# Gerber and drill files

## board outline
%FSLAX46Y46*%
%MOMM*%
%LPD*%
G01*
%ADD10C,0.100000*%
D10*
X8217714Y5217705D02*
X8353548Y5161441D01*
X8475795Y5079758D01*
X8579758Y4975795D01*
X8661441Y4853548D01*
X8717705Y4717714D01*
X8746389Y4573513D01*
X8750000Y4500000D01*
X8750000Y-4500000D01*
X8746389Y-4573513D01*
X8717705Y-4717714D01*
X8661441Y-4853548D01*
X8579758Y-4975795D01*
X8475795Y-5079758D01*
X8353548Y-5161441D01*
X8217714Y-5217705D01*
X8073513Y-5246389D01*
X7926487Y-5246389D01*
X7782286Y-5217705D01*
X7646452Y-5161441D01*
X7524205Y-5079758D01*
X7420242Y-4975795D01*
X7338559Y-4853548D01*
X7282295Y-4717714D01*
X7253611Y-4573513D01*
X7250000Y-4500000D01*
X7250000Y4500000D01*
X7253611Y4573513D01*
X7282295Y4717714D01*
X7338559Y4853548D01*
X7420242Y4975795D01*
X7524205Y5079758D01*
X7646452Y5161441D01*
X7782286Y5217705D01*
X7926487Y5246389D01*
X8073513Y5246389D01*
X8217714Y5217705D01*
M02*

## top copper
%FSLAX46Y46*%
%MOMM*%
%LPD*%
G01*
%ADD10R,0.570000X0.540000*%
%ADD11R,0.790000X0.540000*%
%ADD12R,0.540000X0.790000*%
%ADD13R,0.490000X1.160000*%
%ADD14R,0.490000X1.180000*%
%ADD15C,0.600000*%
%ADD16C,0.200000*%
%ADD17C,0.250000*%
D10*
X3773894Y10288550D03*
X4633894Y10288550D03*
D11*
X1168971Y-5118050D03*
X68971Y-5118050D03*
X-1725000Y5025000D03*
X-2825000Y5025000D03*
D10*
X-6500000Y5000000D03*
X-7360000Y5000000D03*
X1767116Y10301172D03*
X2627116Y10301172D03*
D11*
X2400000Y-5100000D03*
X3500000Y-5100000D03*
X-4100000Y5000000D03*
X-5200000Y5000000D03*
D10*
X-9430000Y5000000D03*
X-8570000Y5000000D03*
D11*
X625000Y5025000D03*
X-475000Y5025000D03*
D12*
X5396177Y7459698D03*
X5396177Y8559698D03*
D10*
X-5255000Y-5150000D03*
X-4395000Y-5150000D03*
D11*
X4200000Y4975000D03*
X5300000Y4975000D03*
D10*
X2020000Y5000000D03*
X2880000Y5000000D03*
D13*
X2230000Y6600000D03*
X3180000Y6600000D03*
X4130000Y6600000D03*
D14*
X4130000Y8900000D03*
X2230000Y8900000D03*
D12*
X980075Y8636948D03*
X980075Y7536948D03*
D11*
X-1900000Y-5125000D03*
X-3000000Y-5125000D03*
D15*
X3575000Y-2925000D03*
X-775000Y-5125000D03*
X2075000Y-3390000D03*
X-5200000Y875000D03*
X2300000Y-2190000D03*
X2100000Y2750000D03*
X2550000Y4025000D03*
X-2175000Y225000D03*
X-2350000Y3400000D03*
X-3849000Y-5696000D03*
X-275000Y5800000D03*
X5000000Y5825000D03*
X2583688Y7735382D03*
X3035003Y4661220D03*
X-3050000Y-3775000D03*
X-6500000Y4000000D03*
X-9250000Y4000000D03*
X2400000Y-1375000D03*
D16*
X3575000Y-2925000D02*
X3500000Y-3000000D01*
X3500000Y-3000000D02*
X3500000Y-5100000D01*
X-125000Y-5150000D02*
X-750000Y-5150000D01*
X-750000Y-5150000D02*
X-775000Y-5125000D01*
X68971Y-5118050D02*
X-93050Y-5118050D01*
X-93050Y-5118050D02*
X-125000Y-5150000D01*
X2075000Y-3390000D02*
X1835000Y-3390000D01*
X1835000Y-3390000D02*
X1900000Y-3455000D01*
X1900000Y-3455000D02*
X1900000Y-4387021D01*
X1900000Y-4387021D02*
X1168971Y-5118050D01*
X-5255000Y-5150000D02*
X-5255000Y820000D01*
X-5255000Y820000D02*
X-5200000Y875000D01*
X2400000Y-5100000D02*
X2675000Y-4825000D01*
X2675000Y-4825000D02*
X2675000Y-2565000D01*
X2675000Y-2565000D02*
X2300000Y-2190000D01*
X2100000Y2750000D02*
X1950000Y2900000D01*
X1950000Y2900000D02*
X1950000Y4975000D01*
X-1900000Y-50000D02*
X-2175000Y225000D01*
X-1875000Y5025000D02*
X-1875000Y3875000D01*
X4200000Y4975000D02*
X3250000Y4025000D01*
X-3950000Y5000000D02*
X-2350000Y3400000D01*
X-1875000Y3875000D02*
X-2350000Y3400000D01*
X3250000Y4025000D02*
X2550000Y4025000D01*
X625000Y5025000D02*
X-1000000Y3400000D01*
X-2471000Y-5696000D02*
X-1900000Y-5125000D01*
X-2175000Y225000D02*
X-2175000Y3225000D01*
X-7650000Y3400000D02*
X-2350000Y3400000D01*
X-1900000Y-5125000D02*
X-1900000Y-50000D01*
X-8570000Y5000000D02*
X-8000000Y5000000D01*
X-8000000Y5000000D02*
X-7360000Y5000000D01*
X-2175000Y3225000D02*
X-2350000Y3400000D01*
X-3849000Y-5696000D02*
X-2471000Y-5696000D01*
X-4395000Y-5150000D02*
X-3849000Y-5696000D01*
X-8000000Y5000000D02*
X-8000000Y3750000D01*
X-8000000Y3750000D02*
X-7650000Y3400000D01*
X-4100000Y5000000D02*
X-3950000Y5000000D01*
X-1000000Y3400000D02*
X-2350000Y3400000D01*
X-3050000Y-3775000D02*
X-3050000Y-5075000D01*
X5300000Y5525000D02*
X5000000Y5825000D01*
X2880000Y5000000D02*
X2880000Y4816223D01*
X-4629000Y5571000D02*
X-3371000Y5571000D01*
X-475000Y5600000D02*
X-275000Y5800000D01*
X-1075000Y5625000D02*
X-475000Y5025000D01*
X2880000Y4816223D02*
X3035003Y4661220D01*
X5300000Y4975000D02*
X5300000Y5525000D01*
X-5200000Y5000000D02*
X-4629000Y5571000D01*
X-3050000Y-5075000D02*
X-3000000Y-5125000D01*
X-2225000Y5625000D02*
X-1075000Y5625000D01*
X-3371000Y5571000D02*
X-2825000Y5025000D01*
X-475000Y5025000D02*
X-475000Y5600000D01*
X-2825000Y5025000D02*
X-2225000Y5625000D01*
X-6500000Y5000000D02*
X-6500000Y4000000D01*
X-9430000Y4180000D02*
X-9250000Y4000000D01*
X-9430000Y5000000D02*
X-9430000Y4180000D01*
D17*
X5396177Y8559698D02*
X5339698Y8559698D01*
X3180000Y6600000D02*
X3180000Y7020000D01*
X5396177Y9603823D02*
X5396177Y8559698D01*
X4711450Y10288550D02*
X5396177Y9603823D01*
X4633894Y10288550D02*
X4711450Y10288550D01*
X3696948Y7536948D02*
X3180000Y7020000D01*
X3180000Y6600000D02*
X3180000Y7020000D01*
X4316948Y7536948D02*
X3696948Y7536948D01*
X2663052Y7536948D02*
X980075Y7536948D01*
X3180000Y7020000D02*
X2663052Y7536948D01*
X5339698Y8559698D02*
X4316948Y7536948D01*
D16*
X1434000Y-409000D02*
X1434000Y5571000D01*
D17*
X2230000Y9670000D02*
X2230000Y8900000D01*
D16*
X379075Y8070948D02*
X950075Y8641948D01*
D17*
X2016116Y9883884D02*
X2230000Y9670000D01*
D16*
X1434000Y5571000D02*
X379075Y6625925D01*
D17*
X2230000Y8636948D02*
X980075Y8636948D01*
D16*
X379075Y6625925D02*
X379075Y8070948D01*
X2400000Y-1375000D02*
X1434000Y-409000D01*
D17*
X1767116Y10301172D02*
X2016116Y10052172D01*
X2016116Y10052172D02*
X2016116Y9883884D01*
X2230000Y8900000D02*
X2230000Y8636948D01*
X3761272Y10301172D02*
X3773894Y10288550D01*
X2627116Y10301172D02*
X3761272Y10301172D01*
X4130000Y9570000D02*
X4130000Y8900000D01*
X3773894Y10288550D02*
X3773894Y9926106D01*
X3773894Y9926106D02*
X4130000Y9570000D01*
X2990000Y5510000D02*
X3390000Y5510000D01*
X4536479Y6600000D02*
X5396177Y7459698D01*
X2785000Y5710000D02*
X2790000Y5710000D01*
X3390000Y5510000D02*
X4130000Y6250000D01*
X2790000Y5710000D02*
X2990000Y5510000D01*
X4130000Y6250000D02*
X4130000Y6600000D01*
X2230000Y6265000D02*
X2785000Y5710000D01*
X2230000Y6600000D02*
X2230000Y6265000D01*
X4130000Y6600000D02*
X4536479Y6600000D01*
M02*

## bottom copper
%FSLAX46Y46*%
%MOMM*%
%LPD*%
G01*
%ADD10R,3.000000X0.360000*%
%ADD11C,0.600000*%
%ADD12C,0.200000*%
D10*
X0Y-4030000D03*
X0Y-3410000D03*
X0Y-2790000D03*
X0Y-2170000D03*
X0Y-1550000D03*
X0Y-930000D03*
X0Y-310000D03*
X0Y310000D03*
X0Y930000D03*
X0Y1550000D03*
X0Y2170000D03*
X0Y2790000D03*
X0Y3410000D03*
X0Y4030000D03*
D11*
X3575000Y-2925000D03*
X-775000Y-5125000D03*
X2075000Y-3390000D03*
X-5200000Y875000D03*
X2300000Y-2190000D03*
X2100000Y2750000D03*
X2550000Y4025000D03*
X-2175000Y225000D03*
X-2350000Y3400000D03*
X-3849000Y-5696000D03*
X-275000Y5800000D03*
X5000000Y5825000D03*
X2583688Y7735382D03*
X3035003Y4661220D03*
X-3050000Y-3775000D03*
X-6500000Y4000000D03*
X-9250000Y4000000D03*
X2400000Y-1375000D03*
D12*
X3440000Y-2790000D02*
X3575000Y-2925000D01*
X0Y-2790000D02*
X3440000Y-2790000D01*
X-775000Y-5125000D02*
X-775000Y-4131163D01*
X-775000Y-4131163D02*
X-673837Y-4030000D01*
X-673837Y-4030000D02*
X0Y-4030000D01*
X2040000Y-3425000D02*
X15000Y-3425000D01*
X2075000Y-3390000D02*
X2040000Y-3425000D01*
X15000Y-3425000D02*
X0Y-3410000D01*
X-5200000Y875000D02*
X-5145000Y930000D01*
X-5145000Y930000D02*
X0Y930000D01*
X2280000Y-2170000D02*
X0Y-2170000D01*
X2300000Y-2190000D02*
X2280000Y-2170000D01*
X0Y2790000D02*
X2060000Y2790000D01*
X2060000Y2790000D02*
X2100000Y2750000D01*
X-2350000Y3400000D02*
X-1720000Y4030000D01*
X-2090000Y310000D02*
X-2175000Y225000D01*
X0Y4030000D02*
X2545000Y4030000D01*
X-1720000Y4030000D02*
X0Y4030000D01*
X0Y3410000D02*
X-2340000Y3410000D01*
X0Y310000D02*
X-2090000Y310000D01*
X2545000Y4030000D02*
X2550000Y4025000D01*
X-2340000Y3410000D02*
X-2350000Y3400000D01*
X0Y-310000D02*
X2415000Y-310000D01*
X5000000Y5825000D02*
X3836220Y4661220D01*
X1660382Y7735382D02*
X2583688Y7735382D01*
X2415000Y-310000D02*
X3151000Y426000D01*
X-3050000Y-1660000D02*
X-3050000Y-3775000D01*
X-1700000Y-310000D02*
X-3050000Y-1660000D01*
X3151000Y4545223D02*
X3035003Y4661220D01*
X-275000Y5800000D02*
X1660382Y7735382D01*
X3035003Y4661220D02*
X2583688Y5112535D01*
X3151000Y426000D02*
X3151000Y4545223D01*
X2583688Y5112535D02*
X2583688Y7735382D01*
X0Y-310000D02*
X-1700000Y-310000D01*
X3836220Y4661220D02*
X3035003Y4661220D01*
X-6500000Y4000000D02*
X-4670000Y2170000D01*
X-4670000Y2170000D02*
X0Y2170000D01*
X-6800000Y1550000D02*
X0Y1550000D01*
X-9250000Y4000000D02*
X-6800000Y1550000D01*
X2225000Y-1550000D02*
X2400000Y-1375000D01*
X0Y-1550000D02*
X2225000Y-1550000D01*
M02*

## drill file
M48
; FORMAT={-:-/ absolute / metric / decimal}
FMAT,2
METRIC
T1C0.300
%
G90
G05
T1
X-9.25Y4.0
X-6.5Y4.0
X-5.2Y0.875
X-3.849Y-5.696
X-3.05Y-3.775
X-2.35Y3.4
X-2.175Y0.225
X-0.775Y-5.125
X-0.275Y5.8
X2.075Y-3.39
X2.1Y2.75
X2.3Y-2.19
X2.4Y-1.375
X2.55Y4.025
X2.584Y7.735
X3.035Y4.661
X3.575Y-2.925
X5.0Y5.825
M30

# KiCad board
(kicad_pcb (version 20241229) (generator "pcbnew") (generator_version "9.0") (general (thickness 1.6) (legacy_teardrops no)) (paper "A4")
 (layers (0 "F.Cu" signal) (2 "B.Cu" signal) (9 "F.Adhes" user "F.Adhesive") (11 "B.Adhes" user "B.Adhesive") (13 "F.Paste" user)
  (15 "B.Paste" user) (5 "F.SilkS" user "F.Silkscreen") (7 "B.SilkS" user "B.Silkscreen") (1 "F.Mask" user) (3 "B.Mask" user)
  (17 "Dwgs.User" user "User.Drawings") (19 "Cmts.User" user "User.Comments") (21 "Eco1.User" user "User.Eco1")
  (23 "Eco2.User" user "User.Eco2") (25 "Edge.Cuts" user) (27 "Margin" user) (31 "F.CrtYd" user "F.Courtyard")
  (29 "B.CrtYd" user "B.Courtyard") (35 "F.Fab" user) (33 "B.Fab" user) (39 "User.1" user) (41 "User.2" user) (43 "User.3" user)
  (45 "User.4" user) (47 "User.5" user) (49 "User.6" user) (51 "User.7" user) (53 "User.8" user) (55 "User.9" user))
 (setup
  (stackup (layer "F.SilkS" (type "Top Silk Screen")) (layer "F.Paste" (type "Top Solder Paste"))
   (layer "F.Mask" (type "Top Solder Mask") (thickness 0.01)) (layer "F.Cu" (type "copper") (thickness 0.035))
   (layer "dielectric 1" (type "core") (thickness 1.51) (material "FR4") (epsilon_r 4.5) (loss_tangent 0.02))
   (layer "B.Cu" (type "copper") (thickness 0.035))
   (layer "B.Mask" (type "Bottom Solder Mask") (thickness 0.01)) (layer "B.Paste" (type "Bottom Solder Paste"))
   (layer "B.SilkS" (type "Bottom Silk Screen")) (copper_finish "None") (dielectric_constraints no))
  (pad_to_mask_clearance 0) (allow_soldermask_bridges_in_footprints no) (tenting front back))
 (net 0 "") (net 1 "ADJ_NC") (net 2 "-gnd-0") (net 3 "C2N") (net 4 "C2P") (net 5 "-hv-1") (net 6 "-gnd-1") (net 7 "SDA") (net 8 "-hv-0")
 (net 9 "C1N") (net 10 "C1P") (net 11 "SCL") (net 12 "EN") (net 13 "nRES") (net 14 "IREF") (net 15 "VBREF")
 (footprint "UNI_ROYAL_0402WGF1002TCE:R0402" (layer "F.Cu") (at 4.203894 -10.28855)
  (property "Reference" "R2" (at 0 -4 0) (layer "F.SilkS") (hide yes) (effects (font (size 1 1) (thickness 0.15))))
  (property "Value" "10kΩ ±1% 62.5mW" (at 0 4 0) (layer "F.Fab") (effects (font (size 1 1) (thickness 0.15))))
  (pad "1" smd rect (at -0.43 0) (size 0.57 0.54) (layers "F.Cu" "F.Mask" "F.Paste") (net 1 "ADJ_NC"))
  (pad "2" smd rect (at 0.43 0) (size 0.57 0.54) (layers "F.Cu" "F.Mask" "F.Paste") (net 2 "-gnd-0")))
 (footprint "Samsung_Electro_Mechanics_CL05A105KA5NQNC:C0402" (layer "F.Cu") (at 0.618971 5.11805 180)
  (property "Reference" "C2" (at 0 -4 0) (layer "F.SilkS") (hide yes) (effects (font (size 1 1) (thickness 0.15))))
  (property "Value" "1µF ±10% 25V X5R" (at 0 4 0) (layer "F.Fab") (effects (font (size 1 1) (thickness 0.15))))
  (pad "1" smd rect (at -0.55 0 180) (size 0.79 0.54) (layers "F.Cu" "F.Mask" "F.Paste") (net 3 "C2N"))
  (pad "2" smd rect (at 0.55 0 180) (size 0.79 0.54) (layers "F.Cu" "F.Mask" "F.Paste") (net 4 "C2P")))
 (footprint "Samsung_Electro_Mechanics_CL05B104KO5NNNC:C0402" (layer "F.Cu") (at -2.275 -5.025 180)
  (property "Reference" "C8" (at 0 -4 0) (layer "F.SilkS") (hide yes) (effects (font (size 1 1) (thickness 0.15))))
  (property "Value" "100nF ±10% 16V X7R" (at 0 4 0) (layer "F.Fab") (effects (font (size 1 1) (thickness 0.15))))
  (pad "1" smd rect (at -0.55 0 180) (size 0.79 0.54) (layers "F.Cu" "F.Mask" "F.Paste") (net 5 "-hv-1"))
  (pad "2" smd rect (at 0.55 0 180) (size 0.79 0.54) (layers "F.Cu" "F.Mask" "F.Paste") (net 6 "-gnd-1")))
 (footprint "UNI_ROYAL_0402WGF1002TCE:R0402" (layer "F.Cu") (at -6.93 -5 180)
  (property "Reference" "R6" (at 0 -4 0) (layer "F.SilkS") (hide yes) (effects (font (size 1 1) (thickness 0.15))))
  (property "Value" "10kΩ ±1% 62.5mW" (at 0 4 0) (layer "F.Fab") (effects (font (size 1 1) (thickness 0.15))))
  (pad "1" smd rect (at -0.43 0 180) (size 0.57 0.54) (layers "F.Cu" "F.Mask" "F.Paste") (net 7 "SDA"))
  (pad "2" smd rect (at 0.43 0 180) (size 0.57 0.54) (layers "F.Cu" "F.Mask" "F.Paste") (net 5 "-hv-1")))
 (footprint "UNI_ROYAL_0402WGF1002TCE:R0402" (layer "F.Cu") (at 2.197116 -10.301172)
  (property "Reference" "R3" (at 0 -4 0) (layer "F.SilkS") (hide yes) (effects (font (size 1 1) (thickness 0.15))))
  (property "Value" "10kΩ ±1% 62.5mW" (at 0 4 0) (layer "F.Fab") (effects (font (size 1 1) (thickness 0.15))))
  (pad "1" smd rect (at -0.43 0) (size 0.57 0.54) (layers "F.Cu" "F.Mask" "F.Paste") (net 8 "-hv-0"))
  (pad "2" smd rect (at 0.43 0) (size 0.57 0.54) (layers "F.Cu" "F.Mask" "F.Paste") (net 1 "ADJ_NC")))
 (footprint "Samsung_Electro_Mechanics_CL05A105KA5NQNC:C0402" (layer "F.Cu") (at 2.95 5.1)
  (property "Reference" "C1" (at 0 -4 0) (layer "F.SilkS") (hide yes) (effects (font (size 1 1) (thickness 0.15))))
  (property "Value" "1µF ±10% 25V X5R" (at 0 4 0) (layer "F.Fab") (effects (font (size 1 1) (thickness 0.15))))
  (pad "1" smd rect (at -0.55 0) (size 0.79 0.54) (layers "F.Cu" "F.Mask" "F.Paste") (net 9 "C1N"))
  (pad "2" smd rect (at 0.55 0) (size 0.79 0.54) (layers "F.Cu" "F.Mask" "F.Paste") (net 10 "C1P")))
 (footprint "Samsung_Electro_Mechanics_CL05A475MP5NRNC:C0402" (layer "F.Cu") (at -4.65 -5 180)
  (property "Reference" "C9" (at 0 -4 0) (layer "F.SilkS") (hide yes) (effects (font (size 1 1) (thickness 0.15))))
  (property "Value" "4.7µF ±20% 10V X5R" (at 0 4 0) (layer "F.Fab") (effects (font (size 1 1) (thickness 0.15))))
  (pad "1" smd rect (at -0.55 0 180) (size 0.79 0.54) (layers "F.Cu" "F.Mask" "F.Paste") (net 5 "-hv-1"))
  (pad "2" smd rect (at 0.55 0 180) (size 0.79 0.54) (layers "F.Cu" "F.Mask" "F.Paste") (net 6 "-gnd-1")))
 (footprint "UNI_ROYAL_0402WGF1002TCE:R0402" (layer "F.Cu") (at -9 -5)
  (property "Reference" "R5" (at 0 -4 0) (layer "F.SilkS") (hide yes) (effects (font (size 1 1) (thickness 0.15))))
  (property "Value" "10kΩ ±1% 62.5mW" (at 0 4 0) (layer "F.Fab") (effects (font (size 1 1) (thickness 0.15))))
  (pad "1" smd rect (at -0.43 0) (size 0.57 0.54) (layers "F.Cu" "F.Mask" "F.Paste") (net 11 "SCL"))
  (pad "2" smd rect (at 0.43 0) (size 0.57 0.54) (layers "F.Cu" "F.Mask" "F.Paste") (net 5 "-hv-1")))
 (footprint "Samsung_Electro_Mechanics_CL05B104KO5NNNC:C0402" (layer "F.Cu") (at 0.075 -5.025 180)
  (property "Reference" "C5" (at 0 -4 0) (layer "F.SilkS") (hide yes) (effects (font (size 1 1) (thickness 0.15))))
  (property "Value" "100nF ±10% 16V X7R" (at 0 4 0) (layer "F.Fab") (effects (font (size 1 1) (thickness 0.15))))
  (pad "1" smd rect (at -0.55 0 180) (size 0.79 0.54) (layers "F.Cu" "F.Mask" "F.Paste") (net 5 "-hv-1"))
  (pad "2" smd rect (at 0.55 0 180) (size 0.79 0.54) (layers "F.Cu" "F.Mask" "F.Paste") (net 6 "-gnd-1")))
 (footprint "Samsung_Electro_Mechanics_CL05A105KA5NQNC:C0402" (layer "F.Cu") (at 5.396177 -8.009698 90)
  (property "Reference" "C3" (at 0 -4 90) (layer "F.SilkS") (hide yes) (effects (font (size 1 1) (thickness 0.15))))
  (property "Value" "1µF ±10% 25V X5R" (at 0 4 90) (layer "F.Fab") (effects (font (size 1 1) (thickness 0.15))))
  (pad "1" smd rect (at -0.55 0 90) (size 0.79 0.54) (layers "F.Cu" "F.Mask" "F.Paste") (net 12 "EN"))
  (pad "2" smd rect (at 0.55 0 90) (size 0.79 0.54) (layers "F.Cu" "F.Mask" "F.Paste") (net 2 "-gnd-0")))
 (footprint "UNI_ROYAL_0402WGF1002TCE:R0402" (layer "F.Cu") (at -4.825 5.15)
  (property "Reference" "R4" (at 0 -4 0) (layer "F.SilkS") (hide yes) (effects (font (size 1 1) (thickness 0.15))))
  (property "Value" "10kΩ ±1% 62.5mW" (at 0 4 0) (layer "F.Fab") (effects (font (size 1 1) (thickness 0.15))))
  (pad "1" smd rect (at -0.43 0) (size 0.57 0.54) (layers "F.Cu" "F.Mask" "F.Paste") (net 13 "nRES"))
  (pad "2" smd rect (at 0.43 0) (size 0.57 0.54) (layers "F.Cu" "F.Mask" "F.Paste") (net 5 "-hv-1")))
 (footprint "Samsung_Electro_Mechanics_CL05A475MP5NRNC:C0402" (layer "F.Cu") (at 4.75 -4.975)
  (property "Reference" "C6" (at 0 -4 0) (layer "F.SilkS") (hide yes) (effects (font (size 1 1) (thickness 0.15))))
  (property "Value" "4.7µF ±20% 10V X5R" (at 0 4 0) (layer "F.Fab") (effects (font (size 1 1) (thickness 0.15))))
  (pad "1" smd rect (at -0.55 0) (size 0.79 0.54) (layers "F.Cu" "F.Mask" "F.Paste") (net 5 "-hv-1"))
  (pad "2" smd rect (at 0.55 0) (size 0.79 0.54) (layers "F.Cu" "F.Mask" "F.Paste") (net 6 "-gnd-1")))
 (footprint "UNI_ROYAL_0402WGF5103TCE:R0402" (layer "F.Cu") (at 2.45 -5)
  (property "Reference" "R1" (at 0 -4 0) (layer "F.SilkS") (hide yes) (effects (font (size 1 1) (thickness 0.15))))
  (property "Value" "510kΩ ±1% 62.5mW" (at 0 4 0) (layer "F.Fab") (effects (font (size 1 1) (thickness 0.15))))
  (pad "1" smd rect (at -0.43 0) (size 0.57 0.54) (layers "F.Cu" "F.Mask" "F.Paste") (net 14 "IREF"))
  (pad "2" smd rect (at 0.43 0) (size 0.57 0.54) (layers "F.Cu" "F.Mask" "F.Paste") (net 6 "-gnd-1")))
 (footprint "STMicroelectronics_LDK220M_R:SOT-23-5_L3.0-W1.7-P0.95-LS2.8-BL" (layer "F.Cu") (at 3.18 -7.75)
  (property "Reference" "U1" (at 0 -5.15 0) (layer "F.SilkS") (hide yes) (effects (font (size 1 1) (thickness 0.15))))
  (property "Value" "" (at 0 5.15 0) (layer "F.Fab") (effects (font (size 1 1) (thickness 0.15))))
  (pad "1" smd rect (at -0.95 1.15) (size 0.49 1.16) (layers "F.Cu" "F.Mask" "F.Paste") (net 12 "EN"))
  (pad "2" smd rect (at 0 1.15) (size 0.49 1.16) (layers "F.Cu" "F.Mask" "F.Paste") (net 2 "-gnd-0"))
  (pad "3" smd rect (at 0.95 1.15) (size 0.49 1.16) (layers "F.Cu" "F.Mask" "F.Paste") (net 12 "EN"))
  (pad "4" smd rect (at 0.95 -1.15) (size 0.49 1.18) (layers "F.Cu" "F.Mask" "F.Paste") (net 1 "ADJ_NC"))
  (pad "5" smd rect (at -0.95 -1.15) (size 0.49 1.18) (layers "F.Cu" "F.Mask" "F.Paste") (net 8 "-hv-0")))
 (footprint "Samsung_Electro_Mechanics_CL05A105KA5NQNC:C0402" (layer "F.Cu") (at 0.980075 -8.086948 -90)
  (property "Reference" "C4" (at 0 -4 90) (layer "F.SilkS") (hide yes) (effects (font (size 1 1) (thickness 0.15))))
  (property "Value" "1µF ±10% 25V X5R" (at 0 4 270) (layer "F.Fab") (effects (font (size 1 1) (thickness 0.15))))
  (pad "1" smd rect (at -0.55 0 270) (size 0.79 0.54) (layers "F.Cu" "F.Mask" "F.Paste") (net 8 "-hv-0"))
  (pad "2" smd rect (at 0.55 0 270) (size 0.79 0.54) (layers "F.Cu" "F.Mask" "F.Paste") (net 2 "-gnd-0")))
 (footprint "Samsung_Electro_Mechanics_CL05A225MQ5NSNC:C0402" (layer "F.Cu") (at -2.45 5.125 180)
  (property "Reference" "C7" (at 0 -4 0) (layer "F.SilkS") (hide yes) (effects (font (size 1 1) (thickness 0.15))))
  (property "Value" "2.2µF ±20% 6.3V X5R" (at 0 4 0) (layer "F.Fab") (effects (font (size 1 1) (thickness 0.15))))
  (pad "1" smd rect (at -0.55 0 180) (size 0.79 0.54) (layers "F.Cu" "F.Mask" "F.Paste") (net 5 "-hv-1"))
  (pad "2" smd rect (at 0.55 0 180) (size 0.79 0.54) (layers "F.Cu" "F.Mask" "F.Paste") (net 6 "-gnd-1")))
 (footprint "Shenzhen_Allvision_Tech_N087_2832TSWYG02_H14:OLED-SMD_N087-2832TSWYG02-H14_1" (layer "F.Cu") (at 0 0)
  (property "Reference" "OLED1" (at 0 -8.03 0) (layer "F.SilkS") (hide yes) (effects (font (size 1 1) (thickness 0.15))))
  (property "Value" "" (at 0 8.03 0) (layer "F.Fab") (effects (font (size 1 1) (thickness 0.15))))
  (fp_poly
   (pts (xy 8.217714 -5.217705) (xy 8.353548 -5.161441) (xy 8.475795 -5.079758) (xy 8.579758 -4.975795) (xy 8.661441 -4.853548)
    (xy 8.717705 -4.717714) (xy 8.746389 -4.573513) (xy 8.75 -4.5) (xy 8.75 4.5) (xy 8.746389 4.573513) (xy 8.717705 4.717714)
    (xy 8.661441 4.853548) (xy 8.579758 4.975795) (xy 8.475795 5.079758) (xy 8.353548 5.161441) (xy 8.217714 5.217705)
    (xy 8.073513 5.246389) (xy 7.926487 5.246389) (xy 7.782286 5.217705) (xy 7.646452 5.161441) (xy 7.524205 5.079758)
    (xy 7.420242 4.975795) (xy 7.338559 4.853548) (xy 7.282295 4.717714) (xy 7.253611 4.573513) (xy 7.25 4.5) (xy 7.25 -4.5)
    (xy 7.253611 -4.573513) (xy 7.282295 -4.717714) (xy 7.338559 -4.853548) (xy 7.420242 -4.975795) (xy 7.524205 -5.079758)
    (xy 7.646452 -5.161441) (xy 7.782286 -5.217705) (xy 7.926487 -5.246389) (xy 8.073513 -5.246389))
   (stroke (width 0.1) (type solid)) (fill no) (layer "Edge.Cuts"))
  (pad "1" smd rect (at 0 4.03) (size 3 0.36) (layers "B.Cu" "B.Mask" "B.Paste") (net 4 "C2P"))
  (pad "2" smd rect (at 0 3.41) (size 3 0.36) (layers "B.Cu" "B.Mask" "B.Paste") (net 3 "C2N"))
  (pad "3" smd rect (at 0 2.79) (size 3 0.36) (layers "B.Cu" "B.Mask" "B.Paste") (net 10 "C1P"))
  (pad "4" smd rect (at 0 2.17) (size 3 0.36) (layers "B.Cu" "B.Mask" "B.Paste") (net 9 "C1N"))
  (pad "5" smd rect (at 0 1.55) (size 3 0.36) (layers "B.Cu" "B.Mask" "B.Paste") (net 8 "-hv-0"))
  (pad "6" smd rect (at 0 0.93) (size 3 0.36) (layers "B.Cu" "B.Mask" "B.Paste") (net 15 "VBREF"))
  (pad "7" smd rect (at 0 0.31) (size 3 0.36) (layers "B.Cu" "B.Mask" "B.Paste") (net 6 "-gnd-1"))
  (pad "8" smd rect (at 0 -0.31) (size 3 0.36) (layers "B.Cu" "B.Mask" "B.Paste") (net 5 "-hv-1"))
  (pad "9" smd rect (at 0 -0.93) (size 3 0.36) (layers "B.Cu" "B.Mask" "B.Paste") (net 13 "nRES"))
  (pad "10" smd rect (at 0 -1.55) (size 3 0.36) (layers "B.Cu" "B.Mask" "B.Paste") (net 11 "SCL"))
  (pad "11" smd rect (at 0 -2.17) (size 3 0.36) (layers "B.Cu" "B.Mask" "B.Paste") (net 7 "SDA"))
  (pad "12" smd rect (at 0 -2.79) (size 3 0.36) (layers "B.Cu" "B.Mask" "B.Paste") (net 14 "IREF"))
  (pad "13" smd rect (at 0 -3.41) (size 3 0.36) (layers "B.Cu" "B.Mask" "B.Paste") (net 5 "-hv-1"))
  (pad "14" smd rect (at 0 -4.03) (size 3 0.36) (layers "B.Cu" "B.Mask" "B.Paste") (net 5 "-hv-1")))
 (segment (start 3.575 2.925) (end 3.5 3) (width 0.2) (layer "F.Cu") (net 10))
 (segment (start 3.5 3) (end 3.5 5.1) (width 0.2) (layer "F.Cu") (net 10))
 (via (at 3.575 2.925) (size 0.6) (drill 0.3) (layers "F.Cu" "B.Cu") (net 10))
 (segment (start 3.44 2.79) (end 3.575 2.925) (width 0.2) (layer "B.Cu") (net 10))
 (segment (start 0 2.79) (end 3.44 2.79) (width 0.2) (layer "B.Cu") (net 10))
 (segment (start -0.125 5.15) (end -0.75 5.15) (width 0.2) (layer "F.Cu") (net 4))
 (segment (start -0.75 5.15) (end -0.775 5.125) (width 0.2) (layer "F.Cu") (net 4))
 (segment (start 0.068971 5.11805) (end -0.09305 5.11805) (width 0.2) (layer "F.Cu") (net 4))
 (segment (start -0.09305 5.11805) (end -0.125 5.15) (width 0.2) (layer "F.Cu") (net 4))
 (via (at -0.775 5.125) (size 0.6) (drill 0.3) (layers "F.Cu" "B.Cu") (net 4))
 (segment (start -0.775 5.125) (end -0.775 4.131163) (width 0.2) (layer "B.Cu") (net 4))
 (segment (start -0.775 4.131163) (end -0.673837 4.03) (width 0.2) (layer "B.Cu") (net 4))
 (segment (start -0.673837 4.03) (end 0 4.03) (width 0.2) (layer "B.Cu") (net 4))
 (segment (start 2.075 3.39) (end 1.835 3.39) (width 0.2) (layer "F.Cu") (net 3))
 (segment (start 1.835 3.39) (end 1.9 3.455) (width 0.2) (layer "F.Cu") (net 3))
 (segment (start 1.9 3.455) (end 1.9 4.387021) (width 0.2) (layer "F.Cu") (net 3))
 (segment (start 1.9 4.387021) (end 1.168971 5.11805) (width 0.2) (layer "F.Cu") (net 3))
 (via (at 2.075 3.39) (size 0.6) (drill 0.3) (layers "F.Cu" "B.Cu") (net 3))
 (segment (start 2.04 3.425) (end 0.015 3.425) (width 0.2) (layer "B.Cu") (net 3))
 (segment (start 2.075 3.39) (end 2.04 3.425) (width 0.2) (layer "B.Cu") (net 3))
 (segment (start 0.015 3.425) (end 0 3.41) (width 0.2) (layer "B.Cu") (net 3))
 (segment (start -5.255 5.15) (end -5.255 -0.82) (width 0.2) (layer "F.Cu") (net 13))
 (segment (start -5.255 -0.82) (end -5.2 -0.875) (width 0.2) (layer "F.Cu") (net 13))
 (via (at -5.2 -0.875) (size 0.6) (drill 0.3) (layers "F.Cu" "B.Cu") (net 13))
 (segment (start -5.2 -0.875) (end -5.145 -0.93) (width 0.2) (layer "B.Cu") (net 13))
 (segment (start -5.145 -0.93) (end 0 -0.93) (width 0.2) (layer "B.Cu") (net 13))
 (segment (start 2.4 5.1) (end 2.675 4.825) (width 0.2) (layer "F.Cu") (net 9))
 (segment (start 2.675 4.825) (end 2.675 2.565) (width 0.2) (layer "F.Cu") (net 9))
 (segment (start 2.675 2.565) (end 2.3 2.19) (width 0.2) (layer "F.Cu") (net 9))
 (via (at 2.3 2.19) (size 0.6) (drill 0.3) (layers "F.Cu" "B.Cu") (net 9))
 (segment (start 2.28 2.17) (end 0 2.17) (width 0.2) (layer "B.Cu") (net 9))
 (segment (start 2.3 2.19) (end 2.28 2.17) (width 0.2) (layer "B.Cu") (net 9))
 (segment (start 2.1 -2.75) (end 1.95 -2.9) (width 0.2) (layer "F.Cu") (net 14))
 (segment (start 1.95 -2.9) (end 1.95 -4.975) (width 0.2) (layer "F.Cu") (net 14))
 (via (at 2.1 -2.75) (size 0.6) (drill 0.3) (layers "F.Cu" "B.Cu") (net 14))
 (segment (start 0 -2.79) (end 2.06 -2.79) (width 0.2) (layer "B.Cu") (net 14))
 (segment (start 2.06 -2.79) (end 2.1 -2.75) (width 0.2) (layer "B.Cu") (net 14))
 (segment (start -1.9 0.05) (end -2.175 -0.225) (width 0.2) (layer "F.Cu") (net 5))
 (segment (start -1.875 -5.025) (end -1.875 -3.875) (width 0.2) (layer "F.Cu") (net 5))
 (segment (start 4.2 -4.975) (end 3.25 -4.025) (width 0.2) (layer "F.Cu") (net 5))
 (segment (start -3.95 -5) (end -2.35 -3.4) (width 0.2) (layer "F.Cu") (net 5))
 (segment (start -1.875 -3.875) (end -2.35 -3.4) (width 0.2) (layer "F.Cu") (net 5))
 (segment (start 3.25 -4.025) (end 2.55 -4.025) (width 0.2) (layer "F.Cu") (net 5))
 (segment (start 0.625 -5.025) (end -1 -3.4) (width 0.2) (layer "F.Cu") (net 5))
 (segment (start -2.471 5.696) (end -1.9 5.125) (width 0.2) (layer "F.Cu") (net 5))
 (segment (start -2.175 -0.225) (end -2.175 -3.225) (width 0.2) (layer "F.Cu") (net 5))
 (segment (start -7.65 -3.4) (end -2.35 -3.4) (width 0.2) (layer "F.Cu") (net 5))
 (segment (start -1.9 5.125) (end -1.9 0.05) (width 0.2) (layer "F.Cu") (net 5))
 (segment (start -8.57 -5) (end -8 -5) (width 0.2) (layer "F.Cu") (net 5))
 (segment (start -8 -5) (end -7.36 -5) (width 0.2) (layer "F.Cu") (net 5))
 (segment (start -2.175 -3.225) (end -2.35 -3.4) (width 0.2) (layer "F.Cu") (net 5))
 (segment (start -3.849 5.696) (end -2.471 5.696) (width 0.2) (layer "F.Cu") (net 5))
 (segment (start -4.395 5.15) (end -3.849 5.696) (width 0.2) (layer "F.Cu") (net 5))
 (segment (start -8 -5) (end -8 -3.75) (width 0.2) (layer "F.Cu") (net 5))
 (segment (start -8 -3.75) (end -7.65 -3.4) (width 0.2) (layer "F.Cu") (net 5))
 (segment (start -4.1 -5) (end -3.95 -5) (width 0.2) (layer "F.Cu") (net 5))
 (segment (start -1 -3.4) (end -2.35 -3.4) (width 0.2) (layer "F.Cu") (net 5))
 (via (at 2.55 -4.025) (size 0.6) (drill 0.3) (layers "F.Cu" "B.Cu") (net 5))
 (via (at -2.175 -0.225) (size 0.6) (drill 0.3) (layers "F.Cu" "B.Cu") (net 5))
 (via (at -2.35 -3.4) (size 0.6) (drill 0.3) (layers "F.Cu" "B.Cu") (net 5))
 (via (at -3.849 5.696) (size 0.6) (drill 0.3) (layers "F.Cu" "B.Cu") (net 5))
 (segment (start -2.35 -3.4) (end -1.72 -4.03) (width 0.2) (layer "B.Cu") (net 5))
 (segment (start -2.09 -0.31) (end -2.175 -0.225) (width 0.2) (layer "B.Cu") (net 5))
 (segment (start 0 -4.03) (end 2.545 -4.03) (width 0.2) (layer "B.Cu") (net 5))
 (segment (start -1.72 -4.03) (end 0 -4.03) (width 0.2) (layer "B.Cu") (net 5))
 (segment (start 0 -3.41) (end -2.34 -3.41) (width 0.2) (layer "B.Cu") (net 5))
 (segment (start 0 -0.31) (end -2.09 -0.31) (width 0.2) (layer "B.Cu") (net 5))
 (segment (start 2.545 -4.03) (end 2.55 -4.025) (width 0.2) (layer "B.Cu") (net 5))
 (segment (start -2.34 -3.41) (end -2.35 -3.4) (width 0.2) (layer "B.Cu") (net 5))
 (segment (start -3.05 3.775) (end -3.05 5.075) (width 0.2) (layer "F.Cu") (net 6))
 (segment (start 5.3 -5.525) (end 5 -5.825) (width 0.2) (layer "F.Cu") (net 6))
 (segment (start 2.88 -5) (end 2.88 -4.816223) (width 0.2) (layer "F.Cu") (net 6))
 (segment (start -4.629 -5.571) (end -3.371 -5.571) (width 0.2) (layer "F.Cu") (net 6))
 (segment (start -0.475 -5.6) (end -0.275 -5.8) (width 0.2) (layer "F.Cu") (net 6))
 (segment (start -1.075 -5.625) (end -0.475 -5.025) (width 0.2) (layer "F.Cu") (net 6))
 (segment (start 2.88 -4.816223) (end 3.035003 -4.66122) (width 0.2) (layer "F.Cu") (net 6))
 (segment (start 5.3 -4.975) (end 5.3 -5.525) (width 0.2) (layer "F.Cu") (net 6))
 (segment (start -5.2 -5) (end -4.629 -5.571) (width 0.2) (layer "F.Cu") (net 6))
 (segment (start -3.05 5.075) (end -3 5.125) (width 0.2) (layer "F.Cu") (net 6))
 (segment (start -2.225 -5.625) (end -1.075 -5.625) (width 0.2) (layer "F.Cu") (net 6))
 (segment (start -3.371 -5.571) (end -2.825 -5.025) (width 0.2) (layer "F.Cu") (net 6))
 (segment (start -0.475 -5.025) (end -0.475 -5.6) (width 0.2) (layer "F.Cu") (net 6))
 (segment (start -2.825 -5.025) (end -2.225 -5.625) (width 0.2) (layer "F.Cu") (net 6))
 (via (at -0.275 -5.8) (size 0.6) (drill 0.3) (layers "F.Cu" "B.Cu") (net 6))
 (via (at 5 -5.825) (size 0.6) (drill 0.3) (layers "F.Cu" "B.Cu") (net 6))
 (via (at 2.583688 -7.735382) (size 0.6) (drill 0.3) (layers "F.Cu" "B.Cu") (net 6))
 (via (at 3.035003 -4.66122) (size 0.6) (drill 0.3) (layers "F.Cu" "B.Cu") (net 6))
 (via (at -3.05 3.775) (size 0.6) (drill 0.3) (layers "F.Cu" "B.Cu") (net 6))
 (segment (start 0 0.31) (end 2.415 0.31) (width 0.2) (layer "B.Cu") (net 6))
 (segment (start 5 -5.825) (end 3.83622 -4.66122) (width 0.2) (layer "B.Cu") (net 6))
 (segment (start 1.660382 -7.735382) (end 2.583688 -7.735382) (width 0.2) (layer "B.Cu") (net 6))
 (segment (start 2.415 0.31) (end 3.151 -0.426) (width 0.2) (layer "B.Cu") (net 6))
 (segment (start -3.05 1.66) (end -3.05 3.775) (width 0.2) (layer "B.Cu") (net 6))
 (segment (start -1.7 0.31) (end -3.05 1.66) (width 0.2) (layer "B.Cu") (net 6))
 (segment (start 3.151 -4.545223) (end 3.035003 -4.66122) (width 0.2) (layer "B.Cu") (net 6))
 (segment (start -0.275 -5.8) (end 1.660382 -7.735382) (width 0.2) (layer "B.Cu") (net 6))
 (segment (start 3.035003 -4.66122) (end 2.583688 -5.112535) (width 0.2) (layer "B.Cu") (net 6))
 (segment (start 3.151 -0.426) (end 3.151 -4.545223) (width 0.2) (layer "B.Cu") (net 6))
 (segment (start 2.583688 -5.112535) (end 2.583688 -7.735382) (width 0.2) (layer "B.Cu") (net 6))
 (segment (start 0 0.31) (end -1.7 0.31) (width 0.2) (layer "B.Cu") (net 6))
 (segment (start 3.83622 -4.66122) (end 3.035003 -4.66122) (width 0.2) (layer "B.Cu") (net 6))
 (segment (start -6.5 -5) (end -6.5 -4) (width 0.2) (layer "F.Cu") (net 7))
 (via (at -6.5 -4) (size 0.6) (drill 0.3) (layers "F.Cu" "B.Cu") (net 7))
 (segment (start -6.5 -4) (end -4.67 -2.17) (width 0.2) (layer "B.Cu") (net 7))
 (segment (start -4.67 -2.17) (end 0 -2.17) (width 0.2) (layer "B.Cu") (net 7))
 (segment (start -9.43 -4.18) (end -9.25 -4) (width 0.2) (layer "F.Cu") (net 11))
 (segment (start -9.43 -5) (end -9.43 -4.18) (width 0.2) (layer "F.Cu") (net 11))
 (via (at -9.25 -4) (size 0.6) (drill 0.3) (layers "F.Cu" "B.Cu") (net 11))
 (segment (start -6.8 -1.55) (end 0 -1.55) (width 0.2) (layer "B.Cu") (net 11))
 (segment (start -9.25 -4) (end -6.8 -1.55) (width 0.2) (layer "B.Cu") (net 11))
 (segment (start 5.396177 -8.559698) (end 5.339698 -8.559698) (width 0.25) (layer "F.Cu") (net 2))
 (segment (start 3.18 -6.6) (end 3.18 -7.02) (width 0.25) (layer "F.Cu") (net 2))
 (segment (start 5.396177 -9.603823) (end 5.396177 -8.559698) (width 0.25) (layer "F.Cu") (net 2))
 (segment (start 4.71145 -10.28855) (end 5.396177 -9.603823) (width 0.25) (layer "F.Cu") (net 2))
 (segment (start 4.633894 -10.28855) (end 4.71145 -10.28855) (width 0.25) (layer "F.Cu") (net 2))
 (segment (start 3.696948 -7.536948) (end 3.18 -7.02) (width 0.25) (layer "F.Cu") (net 2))
 (segment (start 3.18 -6.6) (end 3.18 -7.02) (width 0.25) (layer "F.Cu") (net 2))
 (segment (start 4.316948 -7.536948) (end 3.696948 -7.536948) (width 0.25) (layer "F.Cu") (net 2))
 (segment (start 2.663052 -7.536948) (end 0.980075 -7.536948) (width 0.25) (layer "F.Cu") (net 2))
 (segment (start 3.18 -7.02) (end 2.663052 -7.536948) (width 0.25) (layer "F.Cu") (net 2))
 (segment (start 5.339698 -8.559698) (end 4.316948 -7.536948) (width 0.25) (layer "F.Cu") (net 2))
 (segment (start 1.434 0.409) (end 1.434 -5.571) (width 0.2) (layer "F.Cu") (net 8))
 (segment (start 2.23 -9.67) (end 2.23 -8.9) (width 0.25) (layer "F.Cu") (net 8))
 (segment (start 0.379075 -8.070948) (end 0.950075 -8.641948) (width 0.2) (layer "F.Cu") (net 8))
 (segment (start 2.016116 -9.883884) (end 2.23 -9.67) (width 0.25) (layer "F.Cu") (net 8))
 (segment (start 1.434 -5.571) (end 0.379075 -6.625925) (width 0.2) (layer "F.Cu") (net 8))
 (segment (start 2.23 -8.636948) (end 0.980075 -8.636948) (width 0.25) (layer "F.Cu") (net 8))
 (segment (start 0.379075 -6.625925) (end 0.379075 -8.070948) (width 0.2) (layer "F.Cu") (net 8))
 (segment (start 2.4 1.375) (end 1.434 0.409) (width 0.2) (layer "F.Cu") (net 8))
 (segment (start 1.767116 -10.301172) (end 2.016116 -10.052172) (width 0.25) (layer "F.Cu") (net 8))
 (segment (start 2.016116 -10.052172) (end 2.016116 -9.883884) (width 0.25) (layer "F.Cu") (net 8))
 (segment (start 2.23 -8.9) (end 2.23 -8.636948) (width 0.25) (layer "F.Cu") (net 8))
 (via (at 2.4 1.375) (size 0.6) (drill 0.3) (layers "F.Cu" "B.Cu") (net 8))
 (segment (start 2.225 1.55) (end 2.4 1.375) (width 0.2) (layer "B.Cu") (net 8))
 (segment (start 0 1.55) (end 2.225 1.55) (width 0.2) (layer "B.Cu") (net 8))
 (segment (start 3.761272 -10.301172) (end 3.773894 -10.28855) (width 0.25) (layer "F.Cu") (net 1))
 (segment (start 2.627116 -10.301172) (end 3.761272 -10.301172) (width 0.25) (layer "F.Cu") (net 1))
 (segment (start 4.13 -9.57) (end 4.13 -8.9) (width 0.25) (layer "F.Cu") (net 1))
 (segment (start 3.773894 -10.28855) (end 3.773894 -9.926106) (width 0.25) (layer "F.Cu") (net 1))
 (segment (start 3.773894 -9.926106) (end 4.13 -9.57) (width 0.25) (layer "F.Cu") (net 1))
 (segment (start 2.99 -5.51) (end 3.39 -5.51) (width 0.25) (layer "F.Cu") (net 12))
 (segment (start 4.536479 -6.6) (end 5.396177 -7.459698) (width 0.25) (layer "F.Cu") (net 12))
 (segment (start 2.785 -5.71) (end 2.79 -5.71) (width 0.25) (layer "F.Cu") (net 12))
 (segment (start 3.39 -5.51) (end 4.13 -6.25) (width 0.25) (layer "F.Cu") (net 12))
 (segment (start 2.79 -5.71) (end 2.99 -5.51) (width 0.25) (layer "F.Cu") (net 12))
 (segment (start 4.13 -6.25) (end 4.13 -6.6) (width 0.25) (layer "F.Cu") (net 12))
 (segment (start 2.23 -6.265) (end 2.785 -5.71) (width 0.25) (layer "F.Cu") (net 12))
 (segment (start 2.23 -6.6) (end 2.23 -6.265) (width 0.25) (layer "F.Cu") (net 12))
 (segment (start 4.13 -6.6) (end 4.536479 -6.6) (width 0.25) (layer "F.Cu") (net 12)))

